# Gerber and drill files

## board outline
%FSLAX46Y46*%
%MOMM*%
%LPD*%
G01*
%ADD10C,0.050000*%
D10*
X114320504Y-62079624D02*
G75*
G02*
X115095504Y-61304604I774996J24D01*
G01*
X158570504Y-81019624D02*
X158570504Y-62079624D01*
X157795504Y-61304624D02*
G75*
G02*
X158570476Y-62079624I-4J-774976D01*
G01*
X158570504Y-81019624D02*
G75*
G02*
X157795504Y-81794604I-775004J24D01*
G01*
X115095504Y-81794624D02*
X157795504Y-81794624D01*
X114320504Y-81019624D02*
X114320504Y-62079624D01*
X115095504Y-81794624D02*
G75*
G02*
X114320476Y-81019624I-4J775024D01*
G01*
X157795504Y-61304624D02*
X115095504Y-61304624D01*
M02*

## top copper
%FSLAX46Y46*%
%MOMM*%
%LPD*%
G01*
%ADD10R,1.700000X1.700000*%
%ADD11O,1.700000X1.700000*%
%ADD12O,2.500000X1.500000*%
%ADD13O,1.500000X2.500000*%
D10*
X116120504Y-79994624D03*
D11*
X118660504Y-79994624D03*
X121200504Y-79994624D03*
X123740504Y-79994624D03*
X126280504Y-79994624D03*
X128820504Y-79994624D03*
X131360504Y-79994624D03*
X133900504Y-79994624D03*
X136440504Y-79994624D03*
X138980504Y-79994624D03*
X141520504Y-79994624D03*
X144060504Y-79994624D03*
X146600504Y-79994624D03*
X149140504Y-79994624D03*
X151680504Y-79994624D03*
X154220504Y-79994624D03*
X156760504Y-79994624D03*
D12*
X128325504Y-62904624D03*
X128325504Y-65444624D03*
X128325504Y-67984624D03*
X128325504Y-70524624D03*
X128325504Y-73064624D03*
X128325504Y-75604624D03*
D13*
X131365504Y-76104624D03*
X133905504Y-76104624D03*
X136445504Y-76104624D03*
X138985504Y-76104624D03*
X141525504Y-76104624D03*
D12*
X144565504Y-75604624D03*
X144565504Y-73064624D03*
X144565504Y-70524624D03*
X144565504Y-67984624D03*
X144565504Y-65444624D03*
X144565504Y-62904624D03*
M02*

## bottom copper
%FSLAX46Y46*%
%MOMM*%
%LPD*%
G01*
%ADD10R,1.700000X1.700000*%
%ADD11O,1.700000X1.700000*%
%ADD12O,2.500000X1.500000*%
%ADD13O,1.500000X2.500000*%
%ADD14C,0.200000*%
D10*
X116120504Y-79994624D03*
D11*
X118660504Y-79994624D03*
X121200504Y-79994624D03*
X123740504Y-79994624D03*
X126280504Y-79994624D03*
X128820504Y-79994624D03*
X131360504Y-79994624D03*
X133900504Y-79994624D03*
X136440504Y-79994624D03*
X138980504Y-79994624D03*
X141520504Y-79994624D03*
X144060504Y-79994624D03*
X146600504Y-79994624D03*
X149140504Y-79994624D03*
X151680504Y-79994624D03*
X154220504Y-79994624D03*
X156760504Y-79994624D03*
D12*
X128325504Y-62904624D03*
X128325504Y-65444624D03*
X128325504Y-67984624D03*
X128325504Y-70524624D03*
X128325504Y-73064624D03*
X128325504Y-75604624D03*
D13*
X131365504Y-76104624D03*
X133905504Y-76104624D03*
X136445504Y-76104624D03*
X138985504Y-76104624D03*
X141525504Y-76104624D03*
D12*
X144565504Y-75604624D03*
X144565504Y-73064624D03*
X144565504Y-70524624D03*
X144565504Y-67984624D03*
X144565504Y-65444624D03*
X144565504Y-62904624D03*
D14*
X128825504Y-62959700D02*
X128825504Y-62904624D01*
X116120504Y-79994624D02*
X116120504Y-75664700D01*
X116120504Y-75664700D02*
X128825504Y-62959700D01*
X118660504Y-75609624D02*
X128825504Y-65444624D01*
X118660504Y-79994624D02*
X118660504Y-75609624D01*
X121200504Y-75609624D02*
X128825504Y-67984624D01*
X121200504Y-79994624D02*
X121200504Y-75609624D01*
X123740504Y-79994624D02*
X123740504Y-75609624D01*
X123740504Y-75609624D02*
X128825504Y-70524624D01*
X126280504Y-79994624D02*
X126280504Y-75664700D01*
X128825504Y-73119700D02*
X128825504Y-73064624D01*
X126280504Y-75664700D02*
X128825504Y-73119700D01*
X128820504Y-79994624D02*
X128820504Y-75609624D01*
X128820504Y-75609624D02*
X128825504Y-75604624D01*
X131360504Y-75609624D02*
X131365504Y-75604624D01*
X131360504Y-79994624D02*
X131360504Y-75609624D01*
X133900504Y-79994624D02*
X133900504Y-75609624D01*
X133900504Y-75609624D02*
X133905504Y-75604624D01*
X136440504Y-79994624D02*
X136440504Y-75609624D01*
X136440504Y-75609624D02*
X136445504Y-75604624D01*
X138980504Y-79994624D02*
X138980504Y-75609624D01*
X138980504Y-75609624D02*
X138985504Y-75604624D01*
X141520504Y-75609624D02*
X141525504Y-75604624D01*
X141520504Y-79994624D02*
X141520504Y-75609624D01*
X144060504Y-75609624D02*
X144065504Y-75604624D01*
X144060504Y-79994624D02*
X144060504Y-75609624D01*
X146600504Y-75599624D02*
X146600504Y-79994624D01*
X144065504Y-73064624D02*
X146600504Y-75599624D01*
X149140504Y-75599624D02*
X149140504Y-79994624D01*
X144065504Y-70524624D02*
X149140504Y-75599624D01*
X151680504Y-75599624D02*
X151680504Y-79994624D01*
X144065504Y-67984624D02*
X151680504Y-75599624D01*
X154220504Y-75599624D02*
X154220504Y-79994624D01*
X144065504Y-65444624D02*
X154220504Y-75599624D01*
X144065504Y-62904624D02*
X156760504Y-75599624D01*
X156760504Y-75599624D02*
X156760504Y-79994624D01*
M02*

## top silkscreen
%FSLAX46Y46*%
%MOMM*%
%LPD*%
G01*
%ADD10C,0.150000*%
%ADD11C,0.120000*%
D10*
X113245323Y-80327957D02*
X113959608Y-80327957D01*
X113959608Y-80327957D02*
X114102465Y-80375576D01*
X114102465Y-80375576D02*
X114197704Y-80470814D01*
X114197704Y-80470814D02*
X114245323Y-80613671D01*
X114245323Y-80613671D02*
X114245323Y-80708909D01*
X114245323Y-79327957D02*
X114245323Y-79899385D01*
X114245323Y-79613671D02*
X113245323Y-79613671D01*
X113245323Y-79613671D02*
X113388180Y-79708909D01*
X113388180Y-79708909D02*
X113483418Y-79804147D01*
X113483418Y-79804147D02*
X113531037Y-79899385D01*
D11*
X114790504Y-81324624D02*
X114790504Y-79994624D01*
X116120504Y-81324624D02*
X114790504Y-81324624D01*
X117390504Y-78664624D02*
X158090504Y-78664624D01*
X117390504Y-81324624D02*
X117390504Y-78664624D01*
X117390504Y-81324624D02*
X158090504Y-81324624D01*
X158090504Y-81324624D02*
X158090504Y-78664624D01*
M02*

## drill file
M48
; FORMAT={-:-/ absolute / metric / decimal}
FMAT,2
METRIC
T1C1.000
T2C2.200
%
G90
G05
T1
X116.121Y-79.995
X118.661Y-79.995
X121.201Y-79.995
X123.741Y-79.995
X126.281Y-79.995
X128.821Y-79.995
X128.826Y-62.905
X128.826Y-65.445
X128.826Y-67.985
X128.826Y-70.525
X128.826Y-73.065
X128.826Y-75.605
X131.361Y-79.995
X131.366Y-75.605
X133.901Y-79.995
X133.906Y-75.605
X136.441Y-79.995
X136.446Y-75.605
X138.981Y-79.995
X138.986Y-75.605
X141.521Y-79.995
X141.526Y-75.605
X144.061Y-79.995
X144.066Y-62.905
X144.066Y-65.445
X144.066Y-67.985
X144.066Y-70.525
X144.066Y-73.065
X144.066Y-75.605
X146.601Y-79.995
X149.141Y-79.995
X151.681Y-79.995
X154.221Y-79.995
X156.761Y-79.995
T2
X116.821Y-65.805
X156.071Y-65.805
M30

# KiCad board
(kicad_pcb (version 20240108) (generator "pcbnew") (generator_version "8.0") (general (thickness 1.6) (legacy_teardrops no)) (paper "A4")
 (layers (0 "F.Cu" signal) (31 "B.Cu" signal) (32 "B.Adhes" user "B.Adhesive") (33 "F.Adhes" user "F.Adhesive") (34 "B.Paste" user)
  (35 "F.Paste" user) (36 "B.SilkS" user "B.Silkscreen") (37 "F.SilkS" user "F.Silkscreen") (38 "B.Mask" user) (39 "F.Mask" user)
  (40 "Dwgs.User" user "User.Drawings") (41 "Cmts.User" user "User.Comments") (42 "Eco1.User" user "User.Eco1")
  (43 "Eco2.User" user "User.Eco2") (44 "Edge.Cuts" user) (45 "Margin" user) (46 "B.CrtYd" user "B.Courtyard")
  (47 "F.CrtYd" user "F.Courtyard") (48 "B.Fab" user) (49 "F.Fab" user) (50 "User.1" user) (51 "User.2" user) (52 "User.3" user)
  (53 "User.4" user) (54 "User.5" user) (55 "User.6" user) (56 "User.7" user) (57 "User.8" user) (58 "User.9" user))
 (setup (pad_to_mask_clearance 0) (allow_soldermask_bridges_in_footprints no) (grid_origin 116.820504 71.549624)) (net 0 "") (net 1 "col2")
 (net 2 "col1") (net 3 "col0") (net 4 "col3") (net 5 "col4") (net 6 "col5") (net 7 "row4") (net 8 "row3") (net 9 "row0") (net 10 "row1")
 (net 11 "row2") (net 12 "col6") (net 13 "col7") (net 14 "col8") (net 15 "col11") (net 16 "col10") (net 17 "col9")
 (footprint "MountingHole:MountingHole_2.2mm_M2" (layer "F.Cu") (at 116.820504 65.804624)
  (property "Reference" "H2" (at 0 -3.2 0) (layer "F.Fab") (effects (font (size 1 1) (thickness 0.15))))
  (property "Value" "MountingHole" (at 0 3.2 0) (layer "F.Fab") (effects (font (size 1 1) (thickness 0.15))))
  (pad "" np_thru_hole circle (at 0 0) (size 2.2 2.2) (drill 2.2) (layers "*.Cu" "*.Mask")))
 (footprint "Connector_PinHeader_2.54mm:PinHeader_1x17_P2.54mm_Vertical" (layer "F.Cu") (at 116.120504 79.994624 90)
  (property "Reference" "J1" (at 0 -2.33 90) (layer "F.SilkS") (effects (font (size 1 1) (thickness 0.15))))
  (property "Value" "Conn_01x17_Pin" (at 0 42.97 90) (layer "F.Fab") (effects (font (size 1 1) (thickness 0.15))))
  (fp_line (start -1.33 -1.33) (end 0 -1.33) (stroke (width 0.12) (type solid)) (layer "F.SilkS"))
  (fp_line (start -1.33 0) (end -1.33 -1.33) (stroke (width 0.12) (type solid)) (layer "F.SilkS"))
  (fp_line (start 1.33 1.27) (end 1.33 41.97) (stroke (width 0.12) (type solid)) (layer "F.SilkS"))
  (fp_line (start -1.33 1.27) (end 1.33 1.27) (stroke (width 0.12) (type solid)) (layer "F.SilkS"))
  (fp_line (start -1.33 1.27) (end -1.33 41.97) (stroke (width 0.12) (type solid)) (layer "F.SilkS"))
  (fp_line (start -1.33 41.97) (end 1.33 41.97) (stroke (width 0.12) (type solid)) (layer "F.SilkS"))
  (pad "1" thru_hole rect (at 0 0 90) (size 1.7 1.7) (drill 1) (layers "*.Cu" "*.Mask") (remove_unused_layers no) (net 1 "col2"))
  (pad "2" thru_hole oval (at 0 2.54 90) (size 1.7 1.7) (drill 1) (layers "*.Cu" "*.Mask") (remove_unused_layers no) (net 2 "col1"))
  (pad "3" thru_hole oval (at 0 5.08 90) (size 1.7 1.7) (drill 1) (layers "*.Cu" "*.Mask") (remove_unused_layers no) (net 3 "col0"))
  (pad "4" thru_hole oval (at 0 7.62 90) (size 1.7 1.7) (drill 1) (layers "*.Cu" "*.Mask") (remove_unused_layers no) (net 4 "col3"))
  (pad "5" thru_hole oval (at 0 10.16 90) (size 1.7 1.7) (drill 1) (layers "*.Cu" "*.Mask") (remove_unused_layers no) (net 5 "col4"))
  (pad "6" thru_hole oval (at 0 12.7 90) (size 1.7 1.7) (drill 1) (layers "*.Cu" "*.Mask") (remove_unused_layers no) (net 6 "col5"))
  (pad "7" thru_hole oval (at 0 15.24 90) (size 1.7 1.7) (drill 1) (layers "*.Cu" "*.Mask") (remove_unused_layers no) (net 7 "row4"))
  (pad "8" thru_hole oval (at 0 17.78 90) (size 1.7 1.7) (drill 1) (layers "*.Cu" "*.Mask") (remove_unused_layers no) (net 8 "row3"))
  (pad "9" thru_hole oval (at 0 20.32 90) (size 1.7 1.7) (drill 1) (layers "*.Cu" "*.Mask") (remove_unused_layers no) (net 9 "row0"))
  (pad "10" thru_hole oval (at 0 22.86 90) (size 1.7 1.7) (drill 1) (layers "*.Cu" "*.Mask") (remove_unused_layers no) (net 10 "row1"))
  (pad "11" thru_hole oval (at 0 25.4 90) (size 1.7 1.7) (drill 1) (layers "*.Cu" "*.Mask") (remove_unused_layers no) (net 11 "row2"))
  (pad "12" thru_hole oval (at 0 27.94 90) (size 1.7 1.7) (drill 1) (layers "*.Cu" "*.Mask") (remove_unused_layers no) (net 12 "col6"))
  (pad "13" thru_hole oval (at 0 30.48 90) (size 1.7 1.7) (drill 1) (layers "*.Cu" "*.Mask") (remove_unused_layers no) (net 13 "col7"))
  (pad "14" thru_hole oval (at 0 33.02 90) (size 1.7 1.7) (drill 1) (layers "*.Cu" "*.Mask") (remove_unused_layers no) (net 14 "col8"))
  (pad "15" thru_hole oval (at 0 35.56 90) (size 1.7 1.7) (drill 1) (layers "*.Cu" "*.Mask") (remove_unused_layers no) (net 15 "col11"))
  (pad "16" thru_hole oval (at 0 38.1 90) (size 1.7 1.7) (drill 1) (layers "*.Cu" "*.Mask") (remove_unused_layers no) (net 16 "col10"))
  (pad "17" thru_hole oval (at 0 40.64 90) (size 1.7 1.7) (drill 1) (layers "*.Cu" "*.Mask") (remove_unused_layers no) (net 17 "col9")))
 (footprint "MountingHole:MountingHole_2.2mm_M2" (layer "F.Cu") (at 156.070504 65.804624)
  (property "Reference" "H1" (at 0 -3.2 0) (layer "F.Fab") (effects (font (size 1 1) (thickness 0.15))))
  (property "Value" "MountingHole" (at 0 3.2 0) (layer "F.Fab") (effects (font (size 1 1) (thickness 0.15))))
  (pad "" np_thru_hole circle (at 0 0) (size 2.2 2.2) (drill 2.2) (layers "*.Cu" "*.Mask")))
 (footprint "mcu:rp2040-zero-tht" (layer "B.Cu") (at 136.445504 65.444624 180)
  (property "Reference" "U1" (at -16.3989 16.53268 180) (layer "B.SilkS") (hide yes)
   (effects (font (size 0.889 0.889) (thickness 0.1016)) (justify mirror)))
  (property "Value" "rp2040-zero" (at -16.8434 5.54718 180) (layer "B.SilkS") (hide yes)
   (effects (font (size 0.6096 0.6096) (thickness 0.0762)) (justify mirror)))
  (pad "4" thru_hole oval (at 7.62 2.54) (size 2.5 1.5) (drill 1 (offset -0.5 0)) (layers "*.Cu" "*.Mask") (remove_unused_layers no)
   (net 1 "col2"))
  (pad "5" thru_hole oval (at 7.62 0) (size 2.5 1.5) (drill 1 (offset -0.5 0)) (layers "*.Cu" "*.Mask") (remove_unused_layers no)
   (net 2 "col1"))
  (pad "6" thru_hole oval (at 7.62 -2.54) (size 2.5 1.5) (drill 1 (offset -0.5 0)) (layers "*.Cu" "*.Mask") (remove_unused_layers no)
   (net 3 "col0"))
  (pad "7" thru_hole oval (at 7.62 -5.08) (size 2.5 1.5) (drill 1 (offset -0.5 0)) (layers "*.Cu" "*.Mask") (remove_unused_layers no)
   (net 4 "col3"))
  (pad "8" thru_hole oval (at 7.62 -7.62) (size 2.5 1.5) (drill 1 (offset -0.5 0)) (layers "*.Cu" "*.Mask") (remove_unused_layers no)
   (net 5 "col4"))
  (pad "9" thru_hole oval (at 7.62 -10.16) (size 2.5 1.5) (drill 1 (offset -0.5 0)) (layers "*.Cu" "*.Mask") (remove_unused_layers no)
   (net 6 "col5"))
  (pad "10" thru_hole oval (at 5.08 -10.16 90) (size 2.5 1.5) (drill 1 (offset -0.5 0)) (layers "*.Cu" "*.Mask") (remove_unused_layers no)
   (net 7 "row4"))
  (pad "11" thru_hole oval (at 2.54 -10.16 90) (size 2.5 1.5) (drill 1 (offset -0.5 0)) (layers "*.Cu" "*.Mask") (remove_unused_layers no)
   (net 8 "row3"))
  (pad "12" thru_hole oval (at 0 -10.16 90) (size 2.5 1.5) (drill 1 (offset -0.5 0)) (layers "*.Cu" "*.Mask") (remove_unused_layers no)
   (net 9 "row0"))
  (pad "13" thru_hole oval (at -2.54 -10.16 90) (size 2.5 1.5) (drill 1 (offset -0.5 0)) (layers "*.Cu" "*.Mask") (remove_unused_layers no)
   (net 10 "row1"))
  (pad "14" thru_hole oval (at -5.08 -10.16 90) (size 2.5 1.5) (drill 1 (offset -0.5 0)) (layers "*.Cu" "*.Mask") (remove_unused_layers no)
   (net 11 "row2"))
  (pad "15" thru_hole oval (at -7.62 -10.16 180) (size 2.5 1.5) (drill 1 (offset -0.5 0)) (layers "*.Cu" "*.Mask") (remove_unused_layers no)
   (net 12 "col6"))
  (pad "16" thru_hole oval (at -7.62 -7.62 180) (size 2.5 1.5) (drill 1 (offset -0.5 0)) (layers "*.Cu" "*.Mask") (remove_unused_layers no)
   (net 13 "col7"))
  (pad "17" thru_hole oval (at -7.62 -5.08 180) (size 2.5 1.5) (drill 1 (offset -0.5 0)) (layers "*.Cu" "*.Mask") (remove_unused_layers no)
   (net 14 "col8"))
  (pad "18" thru_hole oval (at -7.62 -2.54 180) (size 2.5 1.5) (drill 1 (offset -0.5 0)) (layers "*.Cu" "*.Mask") (remove_unused_layers no)
   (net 15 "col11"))
  (pad "19" thru_hole oval (at -7.62 0 180) (size 2.5 1.5) (drill 1 (offset -0.5 0)) (layers "*.Cu" "*.Mask") (remove_unused_layers no)
   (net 16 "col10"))
  (pad "20" thru_hole oval (at -7.62 2.54 180) (size 2.5 1.5) (drill 1 (offset -0.5 0)) (layers "*.Cu" "*.Mask") (remove_unused_layers no)
   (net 17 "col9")))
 (gr_arc (start 114.320504 62.079624) (mid 114.547496 61.531616) (end 115.095504 61.304624) (stroke (width 0.05) (type default))
  (layer "Edge.Cuts"))
 (gr_line (start 158.570504 81.019624) (end 158.570504 62.079624) (stroke (width 0.05) (type default)) (layer "Edge.Cuts"))
 (gr_arc (start 157.795504 61.304624) (mid 158.343512 61.531616) (end 158.570504 62.079624) (stroke (width 0.05) (type default))
  (layer "Edge.Cuts"))
 (gr_arc (start 158.570504 81.019624) (mid 158.343512 81.567632) (end 157.795504 81.794624) (stroke (width 0.05) (type default))
  (layer "Edge.Cuts"))
 (gr_line (start 115.095504 81.794624) (end 157.795504 81.794624) (stroke (width 0.05) (type default)) (layer "Edge.Cuts"))
 (gr_line (start 114.320504 81.019624) (end 114.320504 62.079624) (stroke (width 0.05) (type default)) (layer "Edge.Cuts"))
 (gr_arc (start 115.095504 81.794624) (mid 114.547496 81.567632) (end 114.320504 81.019624) (stroke (width 0.05) (type default))
  (layer "Edge.Cuts"))
 (gr_line (start 157.795504 61.304624) (end 115.095504 61.304624) (stroke (width 0.05) (type default)) (layer "Edge.Cuts"))
 (segment (start 128.825504 62.9597) (end 128.825504 62.904624) (width 0.2) (layer "B.Cu") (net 1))
 (segment (start 116.120504 79.994624) (end 116.120504 75.6647) (width 0.2) (layer "B.Cu") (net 1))
 (segment (start 116.120504 75.6647) (end 128.825504 62.9597) (width 0.2) (layer "B.Cu") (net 1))
 (segment (start 118.660504 75.609624) (end 128.825504 65.444624) (width 0.2) (layer "B.Cu") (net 2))
 (segment (start 118.660504 79.994624) (end 118.660504 75.609624) (width 0.2) (layer "B.Cu") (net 2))
 (segment (start 121.200504 75.609624) (end 128.825504 67.984624) (width 0.2) (layer "B.Cu") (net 3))
 (segment (start 121.200504 79.994624) (end 121.200504 75.609624) (width 0.2) (layer "B.Cu") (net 3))
 (segment (start 123.740504 79.994624) (end 123.740504 75.609624) (width 0.2) (layer "B.Cu") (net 4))
 (segment (start 123.740504 75.609624) (end 128.825504 70.524624) (width 0.2) (layer "B.Cu") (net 4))
 (segment (start 126.280504 79.994624) (end 126.280504 75.6647) (width 0.2) (layer "B.Cu") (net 5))
 (segment (start 128.825504 73.1197) (end 128.825504 73.064624) (width 0.2) (layer "B.Cu") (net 5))
 (segment (start 126.280504 75.6647) (end 128.825504 73.1197) (width 0.2) (layer "B.Cu") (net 5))
 (segment (start 128.820504 79.994624) (end 128.820504 75.609624) (width 0.2) (layer "B.Cu") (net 6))
 (segment (start 128.820504 75.609624) (end 128.825504 75.604624) (width 0.2) (layer "B.Cu") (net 6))
 (segment (start 131.360504 75.609624) (end 131.365504 75.604624) (width 0.2) (layer "B.Cu") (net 7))
 (segment (start 131.360504 79.994624) (end 131.360504 75.609624) (width 0.2) (layer "B.Cu") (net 7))
 (segment (start 133.900504 79.994624) (end 133.900504 75.609624) (width 0.2) (layer "B.Cu") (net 8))
 (segment (start 133.900504 75.609624) (end 133.905504 75.604624) (width 0.2) (layer "B.Cu") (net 8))
 (segment (start 136.440504 79.994624) (end 136.440504 75.609624) (width 0.2) (layer "B.Cu") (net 9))
 (segment (start 136.440504 75.609624) (end 136.445504 75.604624) (width 0.2) (layer "B.Cu") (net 9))
 (segment (start 138.980504 79.994624) (end 138.980504 75.609624) (width 0.2) (layer "B.Cu") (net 10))
 (segment (start 138.980504 75.609624) (end 138.985504 75.604624) (width 0.2) (layer "B.Cu") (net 10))
 (segment (start 141.520504 75.609624) (end 141.525504 75.604624) (width 0.2) (layer "B.Cu") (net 11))
 (segment (start 141.520504 79.994624) (end 141.520504 75.609624) (width 0.2) (layer "B.Cu") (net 11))
 (segment (start 144.060504 75.609624) (end 144.065504 75.604624) (width 0.2) (layer "B.Cu") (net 12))
 (segment (start 144.060504 79.994624) (end 144.060504 75.609624) (width 0.2) (layer "B.Cu") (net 12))
 (segment (start 146.600504 75.599624) (end 146.600504 79.994624) (width 0.2) (layer "B.Cu") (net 13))
 (segment (start 144.065504 73.064624) (end 146.600504 75.599624) (width 0.2) (layer "B.Cu") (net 13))
 (segment (start 149.140504 75.599624) (end 149.140504 79.994624) (width 0.2) (layer "B.Cu") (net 14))
 (segment (start 144.065504 70.524624) (end 149.140504 75.599624) (width 0.2) (layer "B.Cu") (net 14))
 (segment (start 151.680504 75.599624) (end 151.680504 79.994624) (width 0.2) (layer "B.Cu") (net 15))
 (segment (start 144.065504 67.984624) (end 151.680504 75.599624) (width 0.2) (layer "B.Cu") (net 15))
 (segment (start 154.220504 75.599624) (end 154.220504 79.994624) (width 0.2) (layer "B.Cu") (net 16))
 (segment (start 144.065504 65.444624) (end 154.220504 75.599624) (width 0.2) (layer "B.Cu") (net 16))
 (segment (start 144.065504 62.904624) (end 156.760504 75.599624) (width 0.2) (layer "B.Cu") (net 17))
 (segment (start 156.760504 75.599624) (end 156.760504 79.994624) (width 0.2) (layer "B.Cu") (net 17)))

